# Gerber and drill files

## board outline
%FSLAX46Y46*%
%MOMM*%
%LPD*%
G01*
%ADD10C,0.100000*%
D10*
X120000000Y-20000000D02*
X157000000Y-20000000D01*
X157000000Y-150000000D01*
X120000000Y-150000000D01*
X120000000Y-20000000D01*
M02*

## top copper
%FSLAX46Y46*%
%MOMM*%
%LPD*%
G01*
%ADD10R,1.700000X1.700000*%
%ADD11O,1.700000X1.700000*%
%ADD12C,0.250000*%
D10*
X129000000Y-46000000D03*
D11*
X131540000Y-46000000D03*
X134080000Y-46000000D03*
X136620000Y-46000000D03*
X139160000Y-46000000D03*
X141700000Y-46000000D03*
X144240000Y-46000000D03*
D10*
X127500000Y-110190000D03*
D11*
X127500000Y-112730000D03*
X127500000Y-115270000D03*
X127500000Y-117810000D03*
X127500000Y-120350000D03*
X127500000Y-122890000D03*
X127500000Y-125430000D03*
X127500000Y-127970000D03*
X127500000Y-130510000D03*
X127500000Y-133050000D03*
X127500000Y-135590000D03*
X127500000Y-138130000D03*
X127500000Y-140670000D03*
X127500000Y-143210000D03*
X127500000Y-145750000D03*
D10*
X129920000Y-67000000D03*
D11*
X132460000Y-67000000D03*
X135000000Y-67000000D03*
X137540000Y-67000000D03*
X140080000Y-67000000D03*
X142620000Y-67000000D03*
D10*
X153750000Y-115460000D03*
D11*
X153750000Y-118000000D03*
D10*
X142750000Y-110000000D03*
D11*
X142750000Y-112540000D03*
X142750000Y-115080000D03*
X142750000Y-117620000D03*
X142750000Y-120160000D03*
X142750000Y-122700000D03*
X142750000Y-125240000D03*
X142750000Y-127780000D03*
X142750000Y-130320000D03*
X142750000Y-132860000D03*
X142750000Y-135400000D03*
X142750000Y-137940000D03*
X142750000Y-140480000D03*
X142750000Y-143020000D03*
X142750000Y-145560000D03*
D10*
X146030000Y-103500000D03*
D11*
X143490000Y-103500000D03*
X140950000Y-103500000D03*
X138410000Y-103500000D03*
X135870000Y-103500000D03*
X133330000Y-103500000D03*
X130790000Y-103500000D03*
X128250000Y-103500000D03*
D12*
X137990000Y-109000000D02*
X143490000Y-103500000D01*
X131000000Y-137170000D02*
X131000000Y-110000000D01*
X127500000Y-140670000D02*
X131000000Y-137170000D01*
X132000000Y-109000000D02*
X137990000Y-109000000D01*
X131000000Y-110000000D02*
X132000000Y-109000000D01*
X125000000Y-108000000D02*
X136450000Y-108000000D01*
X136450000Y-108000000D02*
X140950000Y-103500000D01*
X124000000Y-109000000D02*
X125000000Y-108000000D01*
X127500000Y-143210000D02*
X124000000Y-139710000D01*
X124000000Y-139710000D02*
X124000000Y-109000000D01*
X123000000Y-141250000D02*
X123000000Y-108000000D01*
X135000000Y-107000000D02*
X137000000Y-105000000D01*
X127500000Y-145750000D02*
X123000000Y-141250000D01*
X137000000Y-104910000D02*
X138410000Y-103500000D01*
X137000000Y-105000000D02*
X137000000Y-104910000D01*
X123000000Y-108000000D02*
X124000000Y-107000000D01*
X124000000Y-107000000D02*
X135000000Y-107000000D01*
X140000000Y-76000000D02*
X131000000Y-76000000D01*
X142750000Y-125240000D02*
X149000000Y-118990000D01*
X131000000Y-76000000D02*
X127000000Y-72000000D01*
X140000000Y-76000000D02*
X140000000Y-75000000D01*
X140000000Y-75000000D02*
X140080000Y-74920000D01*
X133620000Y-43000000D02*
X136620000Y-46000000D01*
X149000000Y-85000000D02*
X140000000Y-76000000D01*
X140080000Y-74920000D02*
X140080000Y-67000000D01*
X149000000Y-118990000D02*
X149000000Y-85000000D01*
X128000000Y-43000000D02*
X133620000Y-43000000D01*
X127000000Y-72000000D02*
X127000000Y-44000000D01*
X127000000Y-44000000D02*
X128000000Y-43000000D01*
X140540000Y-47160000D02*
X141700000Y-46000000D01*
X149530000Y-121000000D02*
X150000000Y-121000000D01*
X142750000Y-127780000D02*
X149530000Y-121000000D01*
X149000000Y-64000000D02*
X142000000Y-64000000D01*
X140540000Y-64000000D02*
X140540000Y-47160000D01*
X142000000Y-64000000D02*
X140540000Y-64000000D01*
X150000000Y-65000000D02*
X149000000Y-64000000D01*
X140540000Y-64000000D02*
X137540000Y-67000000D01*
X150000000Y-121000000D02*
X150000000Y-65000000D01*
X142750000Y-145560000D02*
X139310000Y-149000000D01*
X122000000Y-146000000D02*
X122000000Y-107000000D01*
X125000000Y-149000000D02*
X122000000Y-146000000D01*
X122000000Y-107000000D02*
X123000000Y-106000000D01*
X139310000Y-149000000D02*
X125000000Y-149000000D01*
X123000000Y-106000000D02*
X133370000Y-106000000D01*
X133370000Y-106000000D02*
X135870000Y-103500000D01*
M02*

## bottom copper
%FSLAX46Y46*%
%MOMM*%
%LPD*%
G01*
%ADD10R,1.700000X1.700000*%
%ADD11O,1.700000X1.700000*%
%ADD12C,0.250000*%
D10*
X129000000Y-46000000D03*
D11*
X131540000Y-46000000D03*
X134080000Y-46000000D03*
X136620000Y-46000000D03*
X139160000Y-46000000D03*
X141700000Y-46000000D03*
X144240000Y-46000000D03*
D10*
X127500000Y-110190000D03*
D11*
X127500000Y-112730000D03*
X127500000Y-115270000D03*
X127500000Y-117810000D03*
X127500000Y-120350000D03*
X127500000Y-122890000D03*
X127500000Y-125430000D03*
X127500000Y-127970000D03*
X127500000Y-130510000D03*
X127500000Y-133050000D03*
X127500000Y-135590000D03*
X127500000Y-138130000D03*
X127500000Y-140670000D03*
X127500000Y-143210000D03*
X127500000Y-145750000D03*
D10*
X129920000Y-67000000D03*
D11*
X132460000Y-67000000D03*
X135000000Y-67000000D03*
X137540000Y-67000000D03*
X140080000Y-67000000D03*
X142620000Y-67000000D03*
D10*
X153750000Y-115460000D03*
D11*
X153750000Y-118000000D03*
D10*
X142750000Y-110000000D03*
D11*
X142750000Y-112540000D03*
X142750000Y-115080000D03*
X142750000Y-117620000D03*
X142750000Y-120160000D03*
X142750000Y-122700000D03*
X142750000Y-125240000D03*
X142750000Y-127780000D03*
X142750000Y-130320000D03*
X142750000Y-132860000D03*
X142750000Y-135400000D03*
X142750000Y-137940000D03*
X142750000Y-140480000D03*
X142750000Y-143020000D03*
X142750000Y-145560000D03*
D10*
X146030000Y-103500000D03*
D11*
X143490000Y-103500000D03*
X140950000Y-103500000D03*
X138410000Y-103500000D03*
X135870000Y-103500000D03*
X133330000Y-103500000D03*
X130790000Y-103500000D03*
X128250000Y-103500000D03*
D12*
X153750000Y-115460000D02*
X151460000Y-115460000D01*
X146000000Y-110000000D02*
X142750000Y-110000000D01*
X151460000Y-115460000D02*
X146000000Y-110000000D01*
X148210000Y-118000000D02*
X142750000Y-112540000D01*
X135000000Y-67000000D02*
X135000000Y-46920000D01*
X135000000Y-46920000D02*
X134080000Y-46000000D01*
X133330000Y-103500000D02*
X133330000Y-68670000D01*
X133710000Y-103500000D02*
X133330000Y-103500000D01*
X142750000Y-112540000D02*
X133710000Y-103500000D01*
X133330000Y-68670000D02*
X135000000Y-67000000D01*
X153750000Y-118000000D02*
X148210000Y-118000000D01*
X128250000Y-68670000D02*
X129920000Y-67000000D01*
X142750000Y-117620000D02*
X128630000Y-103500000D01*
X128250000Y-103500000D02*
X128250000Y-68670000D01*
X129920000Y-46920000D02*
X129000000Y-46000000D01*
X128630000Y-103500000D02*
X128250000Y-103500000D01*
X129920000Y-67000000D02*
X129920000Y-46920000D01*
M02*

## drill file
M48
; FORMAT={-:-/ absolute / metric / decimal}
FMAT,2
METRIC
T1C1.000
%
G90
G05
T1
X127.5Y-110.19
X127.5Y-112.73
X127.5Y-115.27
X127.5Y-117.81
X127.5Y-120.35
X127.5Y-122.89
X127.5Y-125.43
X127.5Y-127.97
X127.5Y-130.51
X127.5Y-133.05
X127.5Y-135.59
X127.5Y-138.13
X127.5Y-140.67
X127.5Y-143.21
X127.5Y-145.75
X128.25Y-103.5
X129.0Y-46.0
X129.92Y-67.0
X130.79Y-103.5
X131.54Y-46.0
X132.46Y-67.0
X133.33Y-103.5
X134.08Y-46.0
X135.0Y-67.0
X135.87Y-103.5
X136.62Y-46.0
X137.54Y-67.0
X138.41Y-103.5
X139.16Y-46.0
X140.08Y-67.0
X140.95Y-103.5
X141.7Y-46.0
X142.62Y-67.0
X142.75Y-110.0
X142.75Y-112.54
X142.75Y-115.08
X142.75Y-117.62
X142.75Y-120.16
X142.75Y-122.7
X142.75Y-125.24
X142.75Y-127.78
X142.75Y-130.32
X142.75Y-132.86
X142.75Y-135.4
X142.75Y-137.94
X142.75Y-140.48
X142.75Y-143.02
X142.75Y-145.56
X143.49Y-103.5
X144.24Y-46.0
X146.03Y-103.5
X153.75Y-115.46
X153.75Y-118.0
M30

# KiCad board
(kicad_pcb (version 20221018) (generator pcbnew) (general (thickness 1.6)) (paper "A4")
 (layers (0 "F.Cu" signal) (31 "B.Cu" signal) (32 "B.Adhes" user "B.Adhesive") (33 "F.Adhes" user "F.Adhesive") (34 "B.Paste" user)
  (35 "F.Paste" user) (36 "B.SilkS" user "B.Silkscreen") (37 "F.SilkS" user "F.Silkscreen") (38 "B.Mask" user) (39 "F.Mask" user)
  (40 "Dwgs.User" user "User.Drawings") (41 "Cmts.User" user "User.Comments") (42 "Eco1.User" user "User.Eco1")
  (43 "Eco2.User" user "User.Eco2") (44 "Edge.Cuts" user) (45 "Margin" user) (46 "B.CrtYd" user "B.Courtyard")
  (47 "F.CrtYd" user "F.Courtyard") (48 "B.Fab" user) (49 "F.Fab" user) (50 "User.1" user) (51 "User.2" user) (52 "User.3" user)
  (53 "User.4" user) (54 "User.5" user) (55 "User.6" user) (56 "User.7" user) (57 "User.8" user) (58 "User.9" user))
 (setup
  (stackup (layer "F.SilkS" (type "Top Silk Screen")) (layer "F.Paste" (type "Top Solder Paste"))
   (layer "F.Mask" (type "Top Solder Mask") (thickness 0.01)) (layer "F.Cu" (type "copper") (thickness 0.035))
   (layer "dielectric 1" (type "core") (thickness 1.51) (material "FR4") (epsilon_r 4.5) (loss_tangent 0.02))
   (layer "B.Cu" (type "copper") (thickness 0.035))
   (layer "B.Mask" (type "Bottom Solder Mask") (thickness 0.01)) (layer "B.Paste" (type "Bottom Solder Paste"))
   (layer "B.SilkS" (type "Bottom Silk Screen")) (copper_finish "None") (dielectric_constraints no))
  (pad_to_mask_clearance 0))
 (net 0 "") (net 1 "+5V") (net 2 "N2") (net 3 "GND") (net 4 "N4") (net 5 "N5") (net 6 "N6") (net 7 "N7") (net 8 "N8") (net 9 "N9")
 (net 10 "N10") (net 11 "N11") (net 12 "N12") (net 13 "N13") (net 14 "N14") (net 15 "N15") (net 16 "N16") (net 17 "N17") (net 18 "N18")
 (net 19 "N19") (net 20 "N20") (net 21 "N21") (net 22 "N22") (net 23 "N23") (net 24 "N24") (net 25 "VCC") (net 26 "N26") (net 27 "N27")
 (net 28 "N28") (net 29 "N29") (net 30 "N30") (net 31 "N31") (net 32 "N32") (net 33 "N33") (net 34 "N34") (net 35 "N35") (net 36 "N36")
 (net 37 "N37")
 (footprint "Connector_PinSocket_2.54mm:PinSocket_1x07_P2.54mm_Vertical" (layer "F.Cu") (at 129 46 90)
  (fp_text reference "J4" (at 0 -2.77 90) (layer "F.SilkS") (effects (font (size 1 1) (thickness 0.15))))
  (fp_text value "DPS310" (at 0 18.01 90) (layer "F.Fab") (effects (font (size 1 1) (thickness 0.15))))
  (pad "1" thru_hole rect (at 0 0 90) (size 1.7 1.7) (drill 1) (layers "*.Cu" "*.Mask") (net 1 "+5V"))
  (pad "2" thru_hole oval (at 0 2.54 90) (size 1.7 1.7) (drill 1) (layers "*.Cu" "*.Mask") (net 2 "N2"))
  (pad "3" thru_hole oval (at 0 5.08 90) (size 1.7 1.7) (drill 1) (layers "*.Cu" "*.Mask") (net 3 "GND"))
  (pad "4" thru_hole oval (at 0 7.62 90) (size 1.7 1.7) (drill 1) (layers "*.Cu" "*.Mask") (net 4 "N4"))
  (pad "5" thru_hole oval (at 0 10.16 90) (size 1.7 1.7) (drill 1) (layers "*.Cu" "*.Mask") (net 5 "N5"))
  (pad "6" thru_hole oval (at 0 12.7 90) (size 1.7 1.7) (drill 1) (layers "*.Cu" "*.Mask") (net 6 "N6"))
  (pad "7" thru_hole oval (at 0 15.24 90) (size 1.7 1.7) (drill 1) (layers "*.Cu" "*.Mask") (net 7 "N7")))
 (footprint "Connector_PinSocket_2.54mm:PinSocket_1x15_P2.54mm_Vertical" (layer "F.Cu") (at 127.5 110.19)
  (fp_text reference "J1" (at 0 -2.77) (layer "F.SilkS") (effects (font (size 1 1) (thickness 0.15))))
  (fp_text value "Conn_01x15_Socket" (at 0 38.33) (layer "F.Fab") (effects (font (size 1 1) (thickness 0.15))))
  (pad "1" thru_hole rect (at 0 0) (size 1.7 1.7) (drill 1) (layers "*.Cu" "*.Mask") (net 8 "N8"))
  (pad "2" thru_hole oval (at 0 2.54) (size 1.7 1.7) (drill 1) (layers "*.Cu" "*.Mask") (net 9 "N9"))
  (pad "3" thru_hole oval (at 0 5.08) (size 1.7 1.7) (drill 1) (layers "*.Cu" "*.Mask") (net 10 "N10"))
  (pad "4" thru_hole oval (at 0 7.62) (size 1.7 1.7) (drill 1) (layers "*.Cu" "*.Mask") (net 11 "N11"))
  (pad "5" thru_hole oval (at 0 10.16) (size 1.7 1.7) (drill 1) (layers "*.Cu" "*.Mask") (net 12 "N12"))
  (pad "6" thru_hole oval (at 0 12.7) (size 1.7 1.7) (drill 1) (layers "*.Cu" "*.Mask") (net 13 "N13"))
  (pad "7" thru_hole oval (at 0 15.24) (size 1.7 1.7) (drill 1) (layers "*.Cu" "*.Mask") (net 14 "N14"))
  (pad "8" thru_hole oval (at 0 17.78) (size 1.7 1.7) (drill 1) (layers "*.Cu" "*.Mask") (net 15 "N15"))
  (pad "9" thru_hole oval (at 0 20.32) (size 1.7 1.7) (drill 1) (layers "*.Cu" "*.Mask") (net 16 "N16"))
  (pad "10" thru_hole oval (at 0 22.86) (size 1.7 1.7) (drill 1) (layers "*.Cu" "*.Mask") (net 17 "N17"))
  (pad "11" thru_hole oval (at 0 25.4) (size 1.7 1.7) (drill 1) (layers "*.Cu" "*.Mask") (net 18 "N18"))
  (pad "12" thru_hole oval (at 0 27.94) (size 1.7 1.7) (drill 1) (layers "*.Cu" "*.Mask") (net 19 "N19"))
  (pad "13" thru_hole oval (at 0 30.48) (size 1.7 1.7) (drill 1) (layers "*.Cu" "*.Mask") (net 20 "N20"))
  (pad "14" thru_hole oval (at 0 33.02) (size 1.7 1.7) (drill 1) (layers "*.Cu" "*.Mask") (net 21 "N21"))
  (pad "15" thru_hole oval (at 0 35.56) (size 1.7 1.7) (drill 1) (layers "*.Cu" "*.Mask") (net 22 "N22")))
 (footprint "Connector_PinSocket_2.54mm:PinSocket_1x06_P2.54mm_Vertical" (layer "F.Cu") (at 129.92 67 90)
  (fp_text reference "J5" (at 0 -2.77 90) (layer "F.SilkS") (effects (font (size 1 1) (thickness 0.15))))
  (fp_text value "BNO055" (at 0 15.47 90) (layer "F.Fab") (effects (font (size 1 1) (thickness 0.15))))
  (pad "1" thru_hole rect (at 0 0 90) (size 1.7 1.7) (drill 1) (layers "*.Cu" "*.Mask") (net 1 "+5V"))
  (pad "2" thru_hole oval (at 0 2.54 90) (size 1.7 1.7) (drill 1) (layers "*.Cu" "*.Mask") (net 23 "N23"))
  (pad "3" thru_hole oval (at 0 5.08 90) (size 1.7 1.7) (drill 1) (layers "*.Cu" "*.Mask") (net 3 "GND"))
  (pad "4" thru_hole oval (at 0 7.62 90) (size 1.7 1.7) (drill 1) (layers "*.Cu" "*.Mask") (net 6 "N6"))
  (pad "5" thru_hole oval (at 0 10.16 90) (size 1.7 1.7) (drill 1) (layers "*.Cu" "*.Mask") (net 4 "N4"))
  (pad "6" thru_hole oval (at 0 12.7 90) (size 1.7 1.7) (drill 1) (layers "*.Cu" "*.Mask") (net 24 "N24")))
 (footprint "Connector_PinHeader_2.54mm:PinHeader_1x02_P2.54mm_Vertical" (layer "F.Cu") (at 153.75 115.46)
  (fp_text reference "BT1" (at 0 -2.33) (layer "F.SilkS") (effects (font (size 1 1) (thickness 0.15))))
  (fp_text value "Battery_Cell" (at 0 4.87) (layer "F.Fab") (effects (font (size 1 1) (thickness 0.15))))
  (pad "1" thru_hole rect (at 0 0) (size 1.7 1.7) (drill 1) (layers "*.Cu" "*.Mask") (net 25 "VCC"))
  (pad "2" thru_hole oval (at 0 2.54) (size 1.7 1.7) (drill 1) (layers "*.Cu" "*.Mask") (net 3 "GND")))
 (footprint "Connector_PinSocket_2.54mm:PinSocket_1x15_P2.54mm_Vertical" (layer "F.Cu") (at 142.75 110)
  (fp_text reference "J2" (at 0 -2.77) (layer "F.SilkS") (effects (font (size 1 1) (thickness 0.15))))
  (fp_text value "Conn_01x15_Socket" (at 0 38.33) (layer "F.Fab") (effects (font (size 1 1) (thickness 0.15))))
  (pad "1" thru_hole rect (at 0 0) (size 1.7 1.7) (drill 1) (layers "*.Cu" "*.Mask") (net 25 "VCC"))
  (pad "2" thru_hole oval (at 0 2.54) (size 1.7 1.7) (drill 1) (layers "*.Cu" "*.Mask") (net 3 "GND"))
  (pad "3" thru_hole oval (at 0 5.08) (size 1.7 1.7) (drill 1) (layers "*.Cu" "*.Mask") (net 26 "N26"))
  (pad "4" thru_hole oval (at 0 7.62) (size 1.7 1.7) (drill 1) (layers "*.Cu" "*.Mask") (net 1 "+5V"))
  (pad "5" thru_hole oval (at 0 10.16) (size 1.7 1.7) (drill 1) (layers "*.Cu" "*.Mask") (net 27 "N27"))
  (pad "6" thru_hole oval (at 0 12.7) (size 1.7 1.7) (drill 1) (layers "*.Cu" "*.Mask") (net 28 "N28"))
  (pad "7" thru_hole oval (at 0 15.24) (size 1.7 1.7) (drill 1) (layers "*.Cu" "*.Mask") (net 4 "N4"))
  (pad "8" thru_hole oval (at 0 17.78) (size 1.7 1.7) (drill 1) (layers "*.Cu" "*.Mask") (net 6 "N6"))
  (pad "9" thru_hole oval (at 0 20.32) (size 1.7 1.7) (drill 1) (layers "*.Cu" "*.Mask") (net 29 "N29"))
  (pad "10" thru_hole oval (at 0 22.86) (size 1.7 1.7) (drill 1) (layers "*.Cu" "*.Mask") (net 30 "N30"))
  (pad "11" thru_hole oval (at 0 25.4) (size 1.7 1.7) (drill 1) (layers "*.Cu" "*.Mask") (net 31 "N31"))
  (pad "12" thru_hole oval (at 0 27.94) (size 1.7 1.7) (drill 1) (layers "*.Cu" "*.Mask") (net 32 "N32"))
  (pad "13" thru_hole oval (at 0 30.48) (size 1.7 1.7) (drill 1) (layers "*.Cu" "*.Mask") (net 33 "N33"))
  (pad "14" thru_hole oval (at 0 33.02) (size 1.7 1.7) (drill 1) (layers "*.Cu" "*.Mask") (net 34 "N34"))
  (pad "15" thru_hole oval (at 0 35.56) (size 1.7 1.7) (drill 1) (layers "*.Cu" "*.Mask") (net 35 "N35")))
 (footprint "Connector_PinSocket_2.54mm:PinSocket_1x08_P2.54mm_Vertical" (layer "F.Cu") (at 146.03 103.5 -90)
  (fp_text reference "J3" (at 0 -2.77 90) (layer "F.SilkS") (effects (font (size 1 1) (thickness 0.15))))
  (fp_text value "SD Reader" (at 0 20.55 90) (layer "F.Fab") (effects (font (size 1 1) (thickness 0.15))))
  (pad "1" thru_hole rect (at 0 0 270) (size 1.7 1.7) (drill 1) (layers "*.Cu" "*.Mask") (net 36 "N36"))
  (pad "2" thru_hole oval (at 0 2.54 270) (size 1.7 1.7) (drill 1) (layers "*.Cu" "*.Mask") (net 20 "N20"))
  (pad "3" thru_hole oval (at 0 5.08 270) (size 1.7 1.7) (drill 1) (layers "*.Cu" "*.Mask") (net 21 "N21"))
  (pad "4" thru_hole oval (at 0 7.62 270) (size 1.7 1.7) (drill 1) (layers "*.Cu" "*.Mask") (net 22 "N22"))
  (pad "5" thru_hole oval (at 0 10.16 270) (size 1.7 1.7) (drill 1) (layers "*.Cu" "*.Mask") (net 35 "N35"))
  (pad "6" thru_hole oval (at 0 12.7 270) (size 1.7 1.7) (drill 1) (layers "*.Cu" "*.Mask") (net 3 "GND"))
  (pad "7" thru_hole oval (at 0 15.24 270) (size 1.7 1.7) (drill 1) (layers "*.Cu" "*.Mask") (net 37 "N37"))
  (pad "8" thru_hole oval (at 0 17.78 270) (size 1.7 1.7) (drill 1) (layers "*.Cu" "*.Mask") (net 1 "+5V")))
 (gr_rect (start 120 20) (end 157 150) (stroke (width 0.1) (type default)) (fill none) (layer "Edge.Cuts"))
 (segment (start 153.75 115.46) (end 151.46 115.46) (width 0.25) (layer "B.Cu") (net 25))
 (segment (start 146 110) (end 142.75 110) (width 0.25) (layer "B.Cu") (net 25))
 (segment (start 151.46 115.46) (end 146 110) (width 0.25) (layer "B.Cu") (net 25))
 (segment (start 137.99 109) (end 143.49 103.5) (width 0.25) (layer "F.Cu") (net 20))
 (segment (start 131 137.17) (end 131 110) (width 0.25) (layer "F.Cu") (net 20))
 (segment (start 127.5 140.67) (end 131 137.17) (width 0.25) (layer "F.Cu") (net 20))
 (segment (start 132 109) (end 137.99 109) (width 0.25) (layer "F.Cu") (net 20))
 (segment (start 131 110) (end 132 109) (width 0.25) (layer "F.Cu") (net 20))
 (segment (start 125 108) (end 136.45 108) (width 0.25) (layer "F.Cu") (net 21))
 (segment (start 136.45 108) (end 140.95 103.5) (width 0.25) (layer "F.Cu") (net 21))
 (segment (start 124 109) (end 125 108) (width 0.25) (layer "F.Cu") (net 21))
 (segment (start 127.5 143.21) (end 124 139.71) (width 0.25) (layer "F.Cu") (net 21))
 (segment (start 124 139.71) (end 124 109) (width 0.25) (layer "F.Cu") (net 21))
 (segment (start 123 141.25) (end 123 108) (width 0.25) (layer "F.Cu") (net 22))
 (segment (start 135 107) (end 137 105) (width 0.25) (layer "F.Cu") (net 22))
 (segment (start 127.5 145.75) (end 123 141.25) (width 0.25) (layer "F.Cu") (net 22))
 (segment (start 137 104.91) (end 138.41 103.5) (width 0.25) (layer "F.Cu") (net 22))
 (segment (start 137 105) (end 137 104.91) (width 0.25) (layer "F.Cu") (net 22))
 (segment (start 123 108) (end 124 107) (width 0.25) (layer "F.Cu") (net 22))
 (segment (start 124 107) (end 135 107) (width 0.25) (layer "F.Cu") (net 22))
 (segment (start 148.21 118) (end 142.75 112.54) (width 0.25) (layer "B.Cu") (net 3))
 (segment (start 135 67) (end 135 46.92) (width 0.25) (layer "B.Cu") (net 3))
 (segment (start 135 46.92) (end 134.08 46) (width 0.25) (layer "B.Cu") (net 3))
 (segment (start 133.33 103.5) (end 133.33 68.67) (width 0.25) (layer "B.Cu") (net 3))
 (segment (start 133.71 103.5) (end 133.33 103.5) (width 0.25) (layer "B.Cu") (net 3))
 (segment (start 142.75 112.54) (end 133.71 103.5) (width 0.25) (layer "B.Cu") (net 3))
 (segment (start 133.33 68.67) (end 135 67) (width 0.25) (layer "B.Cu") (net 3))
 (segment (start 153.75 118) (end 148.21 118) (width 0.25) (layer "B.Cu") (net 3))
 (segment (start 128.25 68.67) (end 129.92 67) (width 0.25) (layer "B.Cu") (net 1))
 (segment (start 142.75 117.62) (end 128.63 103.5) (width 0.25) (layer "B.Cu") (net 1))
 (segment (start 128.25 103.5) (end 128.25 68.67) (width 0.25) (layer "B.Cu") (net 1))
 (segment (start 129.92 46.92) (end 129 46) (width 0.25) (layer "B.Cu") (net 1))
 (segment (start 128.63 103.5) (end 128.25 103.5) (width 0.25) (layer "B.Cu") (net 1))
 (segment (start 129.92 67) (end 129.92 46.92) (width 0.25) (layer "B.Cu") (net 1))
 (segment (start 140 76) (end 131 76) (width 0.25) (layer "F.Cu") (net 4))
 (segment (start 142.75 125.24) (end 149 118.99) (width 0.25) (layer "F.Cu") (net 4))
 (segment (start 131 76) (end 127 72) (width 0.25) (layer "F.Cu") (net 4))
 (segment (start 140 76) (end 140 75) (width 0.25) (layer "F.Cu") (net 4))
 (segment (start 140 75) (end 140.08 74.92) (width 0.25) (layer "F.Cu") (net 4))
 (segment (start 133.62 43) (end 136.62 46) (width 0.25) (layer "F.Cu") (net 4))
 (segment (start 149 85) (end 140 76) (width 0.25) (layer "F.Cu") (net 4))
 (segment (start 140.08 74.92) (end 140.08 67) (width 0.25) (layer "F.Cu") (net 4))
 (segment (start 149 118.99) (end 149 85) (width 0.25) (layer "F.Cu") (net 4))
 (segment (start 128 43) (end 133.62 43) (width 0.25) (layer "F.Cu") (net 4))
 (segment (start 127 72) (end 127 44) (width 0.25) (layer "F.Cu") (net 4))
 (segment (start 127 44) (end 128 43) (width 0.25) (layer "F.Cu") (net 4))
 (segment (start 140.54 47.16) (end 141.7 46) (width 0.25) (layer "F.Cu") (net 6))
 (segment (start 149.53 121) (end 150 121) (width 0.25) (layer "F.Cu") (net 6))
 (segment (start 142.75 127.78) (end 149.53 121) (width 0.25) (layer "F.Cu") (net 6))
 (segment (start 149 64) (end 142 64) (width 0.25) (layer "F.Cu") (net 6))
 (segment (start 140.54 64) (end 140.54 47.16) (width 0.25) (layer "F.Cu") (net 6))
 (segment (start 142 64) (end 140.54 64) (width 0.25) (layer "F.Cu") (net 6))
 (segment (start 150 65) (end 149 64) (width 0.25) (layer "F.Cu") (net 6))
 (segment (start 140.54 64) (end 137.54 67) (width 0.25) (layer "F.Cu") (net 6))
 (segment (start 150 121) (end 150 65) (width 0.25) (layer "F.Cu") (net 6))
 (segment (start 142.75 145.56) (end 139.31 149) (width 0.25) (layer "F.Cu") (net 35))
 (segment (start 122 146) (end 122 107) (width 0.25) (layer "F.Cu") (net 35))
 (segment (start 125 149) (end 122 146) (width 0.25) (layer "F.Cu") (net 35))
 (segment (start 122 107) (end 123 106) (width 0.25) (layer "F.Cu") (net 35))
 (segment (start 139.31 149) (end 125 149) (width 0.25) (layer "F.Cu") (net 35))
 (segment (start 123 106) (end 133.37 106) (width 0.25) (layer "F.Cu") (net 35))
 (segment (start 133.37 106) (end 135.87 103.5) (width 0.25) (layer "F.Cu") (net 35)))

